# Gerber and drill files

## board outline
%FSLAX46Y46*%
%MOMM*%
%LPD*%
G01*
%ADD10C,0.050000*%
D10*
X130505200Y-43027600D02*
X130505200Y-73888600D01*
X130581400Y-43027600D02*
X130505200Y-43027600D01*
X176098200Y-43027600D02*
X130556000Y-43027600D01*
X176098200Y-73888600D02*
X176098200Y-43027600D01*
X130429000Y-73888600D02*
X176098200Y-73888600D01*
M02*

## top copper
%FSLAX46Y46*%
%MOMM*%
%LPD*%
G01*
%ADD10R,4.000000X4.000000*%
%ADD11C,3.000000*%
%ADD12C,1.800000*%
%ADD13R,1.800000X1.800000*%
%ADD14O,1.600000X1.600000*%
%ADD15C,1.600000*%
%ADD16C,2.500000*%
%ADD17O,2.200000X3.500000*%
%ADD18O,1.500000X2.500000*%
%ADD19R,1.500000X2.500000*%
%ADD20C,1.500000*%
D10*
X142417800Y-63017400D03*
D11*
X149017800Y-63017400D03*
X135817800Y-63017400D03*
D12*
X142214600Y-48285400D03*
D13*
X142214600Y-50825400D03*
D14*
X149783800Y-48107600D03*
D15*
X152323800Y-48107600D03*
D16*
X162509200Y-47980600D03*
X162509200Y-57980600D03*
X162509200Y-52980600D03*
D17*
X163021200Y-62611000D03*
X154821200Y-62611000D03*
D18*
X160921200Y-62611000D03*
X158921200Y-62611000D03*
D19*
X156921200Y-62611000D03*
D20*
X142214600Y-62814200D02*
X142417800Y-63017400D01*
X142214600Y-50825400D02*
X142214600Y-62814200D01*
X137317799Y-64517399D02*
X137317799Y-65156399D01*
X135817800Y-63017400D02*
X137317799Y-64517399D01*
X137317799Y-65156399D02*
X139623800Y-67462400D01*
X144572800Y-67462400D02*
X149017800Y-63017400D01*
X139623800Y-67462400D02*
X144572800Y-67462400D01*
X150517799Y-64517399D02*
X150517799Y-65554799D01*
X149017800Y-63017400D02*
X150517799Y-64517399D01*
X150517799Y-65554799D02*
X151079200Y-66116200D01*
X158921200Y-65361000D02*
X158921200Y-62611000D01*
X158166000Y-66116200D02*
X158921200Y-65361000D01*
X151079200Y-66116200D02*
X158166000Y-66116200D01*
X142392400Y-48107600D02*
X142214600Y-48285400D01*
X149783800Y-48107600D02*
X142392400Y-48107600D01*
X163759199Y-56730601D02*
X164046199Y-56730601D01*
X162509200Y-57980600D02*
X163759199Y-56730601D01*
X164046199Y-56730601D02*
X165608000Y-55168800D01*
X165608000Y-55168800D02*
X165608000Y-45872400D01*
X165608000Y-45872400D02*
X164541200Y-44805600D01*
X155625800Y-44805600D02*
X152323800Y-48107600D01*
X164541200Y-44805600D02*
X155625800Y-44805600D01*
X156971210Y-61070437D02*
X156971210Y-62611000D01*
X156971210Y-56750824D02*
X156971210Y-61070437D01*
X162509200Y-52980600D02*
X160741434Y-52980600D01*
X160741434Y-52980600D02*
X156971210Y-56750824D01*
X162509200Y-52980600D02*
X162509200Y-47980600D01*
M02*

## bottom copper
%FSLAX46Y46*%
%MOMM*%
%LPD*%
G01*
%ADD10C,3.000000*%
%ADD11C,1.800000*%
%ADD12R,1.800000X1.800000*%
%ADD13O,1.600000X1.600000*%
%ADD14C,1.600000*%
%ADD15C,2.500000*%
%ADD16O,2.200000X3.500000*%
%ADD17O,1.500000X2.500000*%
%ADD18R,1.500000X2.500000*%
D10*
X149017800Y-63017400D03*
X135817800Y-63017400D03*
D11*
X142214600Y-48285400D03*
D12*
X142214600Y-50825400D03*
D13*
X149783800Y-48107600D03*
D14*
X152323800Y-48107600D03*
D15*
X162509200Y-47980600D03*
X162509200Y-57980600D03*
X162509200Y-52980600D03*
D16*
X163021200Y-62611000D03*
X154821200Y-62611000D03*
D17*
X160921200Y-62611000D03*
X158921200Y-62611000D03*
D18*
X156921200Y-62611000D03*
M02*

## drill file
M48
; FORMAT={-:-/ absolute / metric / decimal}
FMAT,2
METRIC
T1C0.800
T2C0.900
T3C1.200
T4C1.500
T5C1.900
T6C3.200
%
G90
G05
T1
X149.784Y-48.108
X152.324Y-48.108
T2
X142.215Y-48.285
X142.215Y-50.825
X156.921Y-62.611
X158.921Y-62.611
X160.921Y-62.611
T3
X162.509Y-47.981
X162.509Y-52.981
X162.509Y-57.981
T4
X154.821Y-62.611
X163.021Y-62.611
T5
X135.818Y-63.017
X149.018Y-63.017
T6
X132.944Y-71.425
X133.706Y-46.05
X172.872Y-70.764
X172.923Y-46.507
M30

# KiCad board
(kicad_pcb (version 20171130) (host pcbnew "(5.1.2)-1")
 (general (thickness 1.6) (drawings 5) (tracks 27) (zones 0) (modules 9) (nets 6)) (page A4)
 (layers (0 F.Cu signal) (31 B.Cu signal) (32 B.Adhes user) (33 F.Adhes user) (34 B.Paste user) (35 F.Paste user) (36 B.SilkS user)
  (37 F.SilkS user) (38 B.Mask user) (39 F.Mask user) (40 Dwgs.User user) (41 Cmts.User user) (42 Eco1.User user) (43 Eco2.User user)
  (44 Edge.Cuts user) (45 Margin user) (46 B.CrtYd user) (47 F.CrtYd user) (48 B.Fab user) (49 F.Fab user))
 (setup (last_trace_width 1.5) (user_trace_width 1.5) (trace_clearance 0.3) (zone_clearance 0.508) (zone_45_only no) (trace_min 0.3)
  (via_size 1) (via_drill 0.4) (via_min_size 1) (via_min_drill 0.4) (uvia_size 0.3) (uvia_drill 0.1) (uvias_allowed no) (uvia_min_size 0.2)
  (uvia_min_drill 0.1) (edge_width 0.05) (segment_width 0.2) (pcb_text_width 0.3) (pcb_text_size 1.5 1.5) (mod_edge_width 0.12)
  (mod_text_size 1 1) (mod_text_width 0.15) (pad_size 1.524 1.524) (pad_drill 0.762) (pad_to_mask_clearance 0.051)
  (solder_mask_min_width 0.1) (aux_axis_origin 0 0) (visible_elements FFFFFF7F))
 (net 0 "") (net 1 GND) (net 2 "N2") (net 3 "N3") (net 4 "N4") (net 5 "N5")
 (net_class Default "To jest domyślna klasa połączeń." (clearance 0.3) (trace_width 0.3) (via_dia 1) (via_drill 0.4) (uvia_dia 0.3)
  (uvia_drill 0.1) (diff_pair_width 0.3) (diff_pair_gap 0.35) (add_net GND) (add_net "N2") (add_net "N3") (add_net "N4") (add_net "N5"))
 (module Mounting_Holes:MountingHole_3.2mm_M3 (layer F.Cu) (at 133.7056 46.0502)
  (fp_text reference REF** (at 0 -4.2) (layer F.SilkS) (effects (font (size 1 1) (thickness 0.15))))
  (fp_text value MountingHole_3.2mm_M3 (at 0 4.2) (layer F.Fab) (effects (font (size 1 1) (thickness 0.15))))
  (pad 1 np_thru_hole circle (at 0 0) (size 3.2 3.2) (drill 3.2) (layers *.Cu *.Mask)))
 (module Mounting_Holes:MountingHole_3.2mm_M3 (layer F.Cu) (at 132.9436 71.4248)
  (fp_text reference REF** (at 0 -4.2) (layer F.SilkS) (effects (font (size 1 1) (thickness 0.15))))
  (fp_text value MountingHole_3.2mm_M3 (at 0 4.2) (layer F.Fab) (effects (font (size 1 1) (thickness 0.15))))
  (pad 1 np_thru_hole circle (at 0 0) (size 3.2 3.2) (drill 3.2) (layers *.Cu *.Mask)))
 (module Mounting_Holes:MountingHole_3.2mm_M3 (layer F.Cu) (at 172.8724 70.7644)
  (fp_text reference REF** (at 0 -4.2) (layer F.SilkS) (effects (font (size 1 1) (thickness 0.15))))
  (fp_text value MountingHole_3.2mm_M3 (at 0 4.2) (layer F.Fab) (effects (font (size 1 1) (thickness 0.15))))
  (pad 1 np_thru_hole circle (at 0 0) (size 3.2 3.2) (drill 3.2) (layers *.Cu *.Mask)))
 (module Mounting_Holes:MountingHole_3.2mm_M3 (layer F.Cu) (at 172.9232 46.5074)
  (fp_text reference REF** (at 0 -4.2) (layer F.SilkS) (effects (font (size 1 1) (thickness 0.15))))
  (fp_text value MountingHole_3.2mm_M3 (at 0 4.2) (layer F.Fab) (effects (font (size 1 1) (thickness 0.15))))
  (pad 1 np_thru_hole circle (at 0 0) (size 3.2 3.2) (drill 3.2) (layers *.Cu *.Mask)))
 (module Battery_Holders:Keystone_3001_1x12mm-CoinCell (layer F.Cu) (at 142.4178 63.0174)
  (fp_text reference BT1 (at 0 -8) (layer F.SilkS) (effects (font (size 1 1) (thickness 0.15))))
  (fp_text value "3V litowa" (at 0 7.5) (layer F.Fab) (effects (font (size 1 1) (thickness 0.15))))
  (pad 2 smd rect (at 0 0) (size 4 4) (layers F.Cu F.Mask) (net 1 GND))
  (pad 1 thru_hole circle (at 6.6 0) (size 3 3) (drill 1.9) (layers *.Cu *.Mask) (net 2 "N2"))
  (pad 1 thru_hole circle (at -6.6 0) (size 3 3) (drill 1.9) (layers *.Cu *.Mask) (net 2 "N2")))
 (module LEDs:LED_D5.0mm (layer F.Cu) (at 142.2146 50.8254 90)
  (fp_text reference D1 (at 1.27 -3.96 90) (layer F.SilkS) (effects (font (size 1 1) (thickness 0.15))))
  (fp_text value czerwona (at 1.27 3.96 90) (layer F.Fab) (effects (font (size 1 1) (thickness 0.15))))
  (pad 2 thru_hole circle (at 2.54 0 90) (size 1.8 1.8) (drill 0.9) (layers *.Cu *.Mask) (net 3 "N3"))
  (pad 1 thru_hole rect (at 0 0 90) (size 1.8 1.8) (drill 0.9) (layers *.Cu *.Mask) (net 1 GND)))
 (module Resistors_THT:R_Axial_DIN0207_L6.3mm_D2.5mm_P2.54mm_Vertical (layer F.Cu) (at 152.3238 48.1076 180)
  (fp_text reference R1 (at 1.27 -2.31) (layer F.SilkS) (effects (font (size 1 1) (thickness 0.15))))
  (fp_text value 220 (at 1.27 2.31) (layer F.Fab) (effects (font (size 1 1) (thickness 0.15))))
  (pad 2 thru_hole oval (at 2.54 0 180) (size 1.6 1.6) (drill 0.8) (layers *.Cu *.Mask) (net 3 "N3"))
  (pad 1 thru_hole circle (at 0 0 180) (size 1.6 1.6) (drill 0.8) (layers *.Cu *.Mask) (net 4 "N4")))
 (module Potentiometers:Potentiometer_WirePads (layer F.Cu) (at 162.5092 47.9806)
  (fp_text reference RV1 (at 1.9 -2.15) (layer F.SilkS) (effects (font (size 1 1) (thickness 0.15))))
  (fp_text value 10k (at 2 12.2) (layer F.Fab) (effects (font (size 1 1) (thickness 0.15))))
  (pad 1 thru_hole circle (at 0 0) (size 2.5 2.5) (drill 1.2) (layers *.Cu *.Mask) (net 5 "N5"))
  (pad 3 thru_hole circle (at 0 10) (size 2.5 2.5) (drill 1.2) (layers *.Cu *.Mask) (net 4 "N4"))
  (pad 2 thru_hole circle (at 0 5) (size 2.5 2.5) (drill 1.2) (layers *.Cu *.Mask) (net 5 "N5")))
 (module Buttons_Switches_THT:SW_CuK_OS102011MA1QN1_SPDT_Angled (layer F.Cu) (at 156.9212 62.611)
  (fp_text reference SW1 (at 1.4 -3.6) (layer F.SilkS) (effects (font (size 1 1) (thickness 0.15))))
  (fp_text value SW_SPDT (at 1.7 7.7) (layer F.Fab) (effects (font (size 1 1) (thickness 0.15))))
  (pad "" thru_hole oval (at 6.1 0) (size 2.2 3.5) (drill 1.5) (layers *.Cu *.Mask))
  (pad "" thru_hole oval (at -2.1 0) (size 2.2 3.5) (drill 1.5) (layers *.Cu *.Mask))
  (pad 3 thru_hole oval (at 4 0) (size 1.5 2.5) (drill 0.9) (layers *.Cu *.Mask))
  (pad 2 thru_hole oval (at 2 0) (size 1.5 2.5) (drill 0.9) (layers *.Cu *.Mask) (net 2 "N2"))
  (pad 1 thru_hole rect (at 0 0) (size 1.5 2.5) (drill 0.9) (layers *.Cu *.Mask) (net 5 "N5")))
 (gr_line (start 130.5052 43.0276) (end 130.5052 73.8886) (layer Edge.Cuts) (width 0.05))
 (gr_line (start 130.5814 43.0276) (end 130.5052 43.0276) (layer Edge.Cuts) (width 0.05))
 (gr_line (start 176.0982 43.0276) (end 130.556 43.0276) (layer Edge.Cuts) (width 0.05))
 (gr_line (start 176.0982 73.8886) (end 176.0982 43.0276) (layer Edge.Cuts) (width 0.05))
 (gr_line (start 130.429 73.8886) (end 176.0982 73.8886) (layer Edge.Cuts) (width 0.05))
 (segment (start 142.2146 62.8142) (end 142.4178 63.0174) (width 1.5) (layer F.Cu) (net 1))
 (segment (start 142.2146 50.8254) (end 142.2146 62.8142) (width 1.5) (layer F.Cu) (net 1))
 (segment (start 137.317799 64.517399) (end 137.317799 65.156399) (width 1.5) (layer F.Cu) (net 2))
 (segment (start 135.8178 63.0174) (end 137.317799 64.517399) (width 1.5) (layer F.Cu) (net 2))
 (segment (start 137.317799 65.156399) (end 139.6238 67.4624) (width 1.5) (layer F.Cu) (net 2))
 (segment (start 144.5728 67.4624) (end 149.0178 63.0174) (width 1.5) (layer F.Cu) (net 2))
 (segment (start 139.6238 67.4624) (end 144.5728 67.4624) (width 1.5) (layer F.Cu) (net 2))
 (segment (start 150.517799 64.517399) (end 150.517799 65.554799) (width 1.5) (layer F.Cu) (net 2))
 (segment (start 149.0178 63.0174) (end 150.517799 64.517399) (width 1.5) (layer F.Cu) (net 2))
 (segment (start 150.517799 65.554799) (end 151.0792 66.1162) (width 1.5) (layer F.Cu) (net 2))
 (segment (start 158.9212 65.361) (end 158.9212 62.611) (width 1.5) (layer F.Cu) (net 2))
 (segment (start 158.166 66.1162) (end 158.9212 65.361) (width 1.5) (layer F.Cu) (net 2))
 (segment (start 151.0792 66.1162) (end 158.166 66.1162) (width 1.5) (layer F.Cu) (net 2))
 (segment (start 142.3924 48.1076) (end 142.2146 48.2854) (width 1.5) (layer F.Cu) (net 3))
 (segment (start 149.7838 48.1076) (end 142.3924 48.1076) (width 1.5) (layer F.Cu) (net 3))
 (segment (start 163.759199 56.730601) (end 164.046199 56.730601) (width 1.5) (layer F.Cu) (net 4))
 (segment (start 162.5092 57.9806) (end 163.759199 56.730601) (width 1.5) (layer F.Cu) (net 4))
 (segment (start 164.046199 56.730601) (end 165.608 55.1688) (width 1.5) (layer F.Cu) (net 4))
 (segment (start 165.608 55.1688) (end 165.608 45.8724) (width 1.5) (layer F.Cu) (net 4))
 (segment (start 165.608 45.8724) (end 164.5412 44.8056) (width 1.5) (layer F.Cu) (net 4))
 (segment (start 155.6258 44.8056) (end 152.3238 48.1076) (width 1.5) (layer F.Cu) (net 4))
 (segment (start 164.5412 44.8056) (end 155.6258 44.8056) (width 1.5) (layer F.Cu) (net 4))
 (segment (start 156.97121 61.070437) (end 156.97121 62.611) (width 1.5) (layer F.Cu) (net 5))
 (segment (start 156.97121 56.750824) (end 156.97121 61.070437) (width 1.5) (layer F.Cu) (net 5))
 (segment (start 162.5092 52.9806) (end 160.741434 52.9806) (width 1.5) (layer F.Cu) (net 5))
 (segment (start 160.741434 52.9806) (end 156.97121 56.750824) (width 1.5) (layer F.Cu) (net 5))
 (segment (start 162.5092 52.9806) (end 162.5092 47.9806) (width 1.5) (layer F.Cu) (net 5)))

